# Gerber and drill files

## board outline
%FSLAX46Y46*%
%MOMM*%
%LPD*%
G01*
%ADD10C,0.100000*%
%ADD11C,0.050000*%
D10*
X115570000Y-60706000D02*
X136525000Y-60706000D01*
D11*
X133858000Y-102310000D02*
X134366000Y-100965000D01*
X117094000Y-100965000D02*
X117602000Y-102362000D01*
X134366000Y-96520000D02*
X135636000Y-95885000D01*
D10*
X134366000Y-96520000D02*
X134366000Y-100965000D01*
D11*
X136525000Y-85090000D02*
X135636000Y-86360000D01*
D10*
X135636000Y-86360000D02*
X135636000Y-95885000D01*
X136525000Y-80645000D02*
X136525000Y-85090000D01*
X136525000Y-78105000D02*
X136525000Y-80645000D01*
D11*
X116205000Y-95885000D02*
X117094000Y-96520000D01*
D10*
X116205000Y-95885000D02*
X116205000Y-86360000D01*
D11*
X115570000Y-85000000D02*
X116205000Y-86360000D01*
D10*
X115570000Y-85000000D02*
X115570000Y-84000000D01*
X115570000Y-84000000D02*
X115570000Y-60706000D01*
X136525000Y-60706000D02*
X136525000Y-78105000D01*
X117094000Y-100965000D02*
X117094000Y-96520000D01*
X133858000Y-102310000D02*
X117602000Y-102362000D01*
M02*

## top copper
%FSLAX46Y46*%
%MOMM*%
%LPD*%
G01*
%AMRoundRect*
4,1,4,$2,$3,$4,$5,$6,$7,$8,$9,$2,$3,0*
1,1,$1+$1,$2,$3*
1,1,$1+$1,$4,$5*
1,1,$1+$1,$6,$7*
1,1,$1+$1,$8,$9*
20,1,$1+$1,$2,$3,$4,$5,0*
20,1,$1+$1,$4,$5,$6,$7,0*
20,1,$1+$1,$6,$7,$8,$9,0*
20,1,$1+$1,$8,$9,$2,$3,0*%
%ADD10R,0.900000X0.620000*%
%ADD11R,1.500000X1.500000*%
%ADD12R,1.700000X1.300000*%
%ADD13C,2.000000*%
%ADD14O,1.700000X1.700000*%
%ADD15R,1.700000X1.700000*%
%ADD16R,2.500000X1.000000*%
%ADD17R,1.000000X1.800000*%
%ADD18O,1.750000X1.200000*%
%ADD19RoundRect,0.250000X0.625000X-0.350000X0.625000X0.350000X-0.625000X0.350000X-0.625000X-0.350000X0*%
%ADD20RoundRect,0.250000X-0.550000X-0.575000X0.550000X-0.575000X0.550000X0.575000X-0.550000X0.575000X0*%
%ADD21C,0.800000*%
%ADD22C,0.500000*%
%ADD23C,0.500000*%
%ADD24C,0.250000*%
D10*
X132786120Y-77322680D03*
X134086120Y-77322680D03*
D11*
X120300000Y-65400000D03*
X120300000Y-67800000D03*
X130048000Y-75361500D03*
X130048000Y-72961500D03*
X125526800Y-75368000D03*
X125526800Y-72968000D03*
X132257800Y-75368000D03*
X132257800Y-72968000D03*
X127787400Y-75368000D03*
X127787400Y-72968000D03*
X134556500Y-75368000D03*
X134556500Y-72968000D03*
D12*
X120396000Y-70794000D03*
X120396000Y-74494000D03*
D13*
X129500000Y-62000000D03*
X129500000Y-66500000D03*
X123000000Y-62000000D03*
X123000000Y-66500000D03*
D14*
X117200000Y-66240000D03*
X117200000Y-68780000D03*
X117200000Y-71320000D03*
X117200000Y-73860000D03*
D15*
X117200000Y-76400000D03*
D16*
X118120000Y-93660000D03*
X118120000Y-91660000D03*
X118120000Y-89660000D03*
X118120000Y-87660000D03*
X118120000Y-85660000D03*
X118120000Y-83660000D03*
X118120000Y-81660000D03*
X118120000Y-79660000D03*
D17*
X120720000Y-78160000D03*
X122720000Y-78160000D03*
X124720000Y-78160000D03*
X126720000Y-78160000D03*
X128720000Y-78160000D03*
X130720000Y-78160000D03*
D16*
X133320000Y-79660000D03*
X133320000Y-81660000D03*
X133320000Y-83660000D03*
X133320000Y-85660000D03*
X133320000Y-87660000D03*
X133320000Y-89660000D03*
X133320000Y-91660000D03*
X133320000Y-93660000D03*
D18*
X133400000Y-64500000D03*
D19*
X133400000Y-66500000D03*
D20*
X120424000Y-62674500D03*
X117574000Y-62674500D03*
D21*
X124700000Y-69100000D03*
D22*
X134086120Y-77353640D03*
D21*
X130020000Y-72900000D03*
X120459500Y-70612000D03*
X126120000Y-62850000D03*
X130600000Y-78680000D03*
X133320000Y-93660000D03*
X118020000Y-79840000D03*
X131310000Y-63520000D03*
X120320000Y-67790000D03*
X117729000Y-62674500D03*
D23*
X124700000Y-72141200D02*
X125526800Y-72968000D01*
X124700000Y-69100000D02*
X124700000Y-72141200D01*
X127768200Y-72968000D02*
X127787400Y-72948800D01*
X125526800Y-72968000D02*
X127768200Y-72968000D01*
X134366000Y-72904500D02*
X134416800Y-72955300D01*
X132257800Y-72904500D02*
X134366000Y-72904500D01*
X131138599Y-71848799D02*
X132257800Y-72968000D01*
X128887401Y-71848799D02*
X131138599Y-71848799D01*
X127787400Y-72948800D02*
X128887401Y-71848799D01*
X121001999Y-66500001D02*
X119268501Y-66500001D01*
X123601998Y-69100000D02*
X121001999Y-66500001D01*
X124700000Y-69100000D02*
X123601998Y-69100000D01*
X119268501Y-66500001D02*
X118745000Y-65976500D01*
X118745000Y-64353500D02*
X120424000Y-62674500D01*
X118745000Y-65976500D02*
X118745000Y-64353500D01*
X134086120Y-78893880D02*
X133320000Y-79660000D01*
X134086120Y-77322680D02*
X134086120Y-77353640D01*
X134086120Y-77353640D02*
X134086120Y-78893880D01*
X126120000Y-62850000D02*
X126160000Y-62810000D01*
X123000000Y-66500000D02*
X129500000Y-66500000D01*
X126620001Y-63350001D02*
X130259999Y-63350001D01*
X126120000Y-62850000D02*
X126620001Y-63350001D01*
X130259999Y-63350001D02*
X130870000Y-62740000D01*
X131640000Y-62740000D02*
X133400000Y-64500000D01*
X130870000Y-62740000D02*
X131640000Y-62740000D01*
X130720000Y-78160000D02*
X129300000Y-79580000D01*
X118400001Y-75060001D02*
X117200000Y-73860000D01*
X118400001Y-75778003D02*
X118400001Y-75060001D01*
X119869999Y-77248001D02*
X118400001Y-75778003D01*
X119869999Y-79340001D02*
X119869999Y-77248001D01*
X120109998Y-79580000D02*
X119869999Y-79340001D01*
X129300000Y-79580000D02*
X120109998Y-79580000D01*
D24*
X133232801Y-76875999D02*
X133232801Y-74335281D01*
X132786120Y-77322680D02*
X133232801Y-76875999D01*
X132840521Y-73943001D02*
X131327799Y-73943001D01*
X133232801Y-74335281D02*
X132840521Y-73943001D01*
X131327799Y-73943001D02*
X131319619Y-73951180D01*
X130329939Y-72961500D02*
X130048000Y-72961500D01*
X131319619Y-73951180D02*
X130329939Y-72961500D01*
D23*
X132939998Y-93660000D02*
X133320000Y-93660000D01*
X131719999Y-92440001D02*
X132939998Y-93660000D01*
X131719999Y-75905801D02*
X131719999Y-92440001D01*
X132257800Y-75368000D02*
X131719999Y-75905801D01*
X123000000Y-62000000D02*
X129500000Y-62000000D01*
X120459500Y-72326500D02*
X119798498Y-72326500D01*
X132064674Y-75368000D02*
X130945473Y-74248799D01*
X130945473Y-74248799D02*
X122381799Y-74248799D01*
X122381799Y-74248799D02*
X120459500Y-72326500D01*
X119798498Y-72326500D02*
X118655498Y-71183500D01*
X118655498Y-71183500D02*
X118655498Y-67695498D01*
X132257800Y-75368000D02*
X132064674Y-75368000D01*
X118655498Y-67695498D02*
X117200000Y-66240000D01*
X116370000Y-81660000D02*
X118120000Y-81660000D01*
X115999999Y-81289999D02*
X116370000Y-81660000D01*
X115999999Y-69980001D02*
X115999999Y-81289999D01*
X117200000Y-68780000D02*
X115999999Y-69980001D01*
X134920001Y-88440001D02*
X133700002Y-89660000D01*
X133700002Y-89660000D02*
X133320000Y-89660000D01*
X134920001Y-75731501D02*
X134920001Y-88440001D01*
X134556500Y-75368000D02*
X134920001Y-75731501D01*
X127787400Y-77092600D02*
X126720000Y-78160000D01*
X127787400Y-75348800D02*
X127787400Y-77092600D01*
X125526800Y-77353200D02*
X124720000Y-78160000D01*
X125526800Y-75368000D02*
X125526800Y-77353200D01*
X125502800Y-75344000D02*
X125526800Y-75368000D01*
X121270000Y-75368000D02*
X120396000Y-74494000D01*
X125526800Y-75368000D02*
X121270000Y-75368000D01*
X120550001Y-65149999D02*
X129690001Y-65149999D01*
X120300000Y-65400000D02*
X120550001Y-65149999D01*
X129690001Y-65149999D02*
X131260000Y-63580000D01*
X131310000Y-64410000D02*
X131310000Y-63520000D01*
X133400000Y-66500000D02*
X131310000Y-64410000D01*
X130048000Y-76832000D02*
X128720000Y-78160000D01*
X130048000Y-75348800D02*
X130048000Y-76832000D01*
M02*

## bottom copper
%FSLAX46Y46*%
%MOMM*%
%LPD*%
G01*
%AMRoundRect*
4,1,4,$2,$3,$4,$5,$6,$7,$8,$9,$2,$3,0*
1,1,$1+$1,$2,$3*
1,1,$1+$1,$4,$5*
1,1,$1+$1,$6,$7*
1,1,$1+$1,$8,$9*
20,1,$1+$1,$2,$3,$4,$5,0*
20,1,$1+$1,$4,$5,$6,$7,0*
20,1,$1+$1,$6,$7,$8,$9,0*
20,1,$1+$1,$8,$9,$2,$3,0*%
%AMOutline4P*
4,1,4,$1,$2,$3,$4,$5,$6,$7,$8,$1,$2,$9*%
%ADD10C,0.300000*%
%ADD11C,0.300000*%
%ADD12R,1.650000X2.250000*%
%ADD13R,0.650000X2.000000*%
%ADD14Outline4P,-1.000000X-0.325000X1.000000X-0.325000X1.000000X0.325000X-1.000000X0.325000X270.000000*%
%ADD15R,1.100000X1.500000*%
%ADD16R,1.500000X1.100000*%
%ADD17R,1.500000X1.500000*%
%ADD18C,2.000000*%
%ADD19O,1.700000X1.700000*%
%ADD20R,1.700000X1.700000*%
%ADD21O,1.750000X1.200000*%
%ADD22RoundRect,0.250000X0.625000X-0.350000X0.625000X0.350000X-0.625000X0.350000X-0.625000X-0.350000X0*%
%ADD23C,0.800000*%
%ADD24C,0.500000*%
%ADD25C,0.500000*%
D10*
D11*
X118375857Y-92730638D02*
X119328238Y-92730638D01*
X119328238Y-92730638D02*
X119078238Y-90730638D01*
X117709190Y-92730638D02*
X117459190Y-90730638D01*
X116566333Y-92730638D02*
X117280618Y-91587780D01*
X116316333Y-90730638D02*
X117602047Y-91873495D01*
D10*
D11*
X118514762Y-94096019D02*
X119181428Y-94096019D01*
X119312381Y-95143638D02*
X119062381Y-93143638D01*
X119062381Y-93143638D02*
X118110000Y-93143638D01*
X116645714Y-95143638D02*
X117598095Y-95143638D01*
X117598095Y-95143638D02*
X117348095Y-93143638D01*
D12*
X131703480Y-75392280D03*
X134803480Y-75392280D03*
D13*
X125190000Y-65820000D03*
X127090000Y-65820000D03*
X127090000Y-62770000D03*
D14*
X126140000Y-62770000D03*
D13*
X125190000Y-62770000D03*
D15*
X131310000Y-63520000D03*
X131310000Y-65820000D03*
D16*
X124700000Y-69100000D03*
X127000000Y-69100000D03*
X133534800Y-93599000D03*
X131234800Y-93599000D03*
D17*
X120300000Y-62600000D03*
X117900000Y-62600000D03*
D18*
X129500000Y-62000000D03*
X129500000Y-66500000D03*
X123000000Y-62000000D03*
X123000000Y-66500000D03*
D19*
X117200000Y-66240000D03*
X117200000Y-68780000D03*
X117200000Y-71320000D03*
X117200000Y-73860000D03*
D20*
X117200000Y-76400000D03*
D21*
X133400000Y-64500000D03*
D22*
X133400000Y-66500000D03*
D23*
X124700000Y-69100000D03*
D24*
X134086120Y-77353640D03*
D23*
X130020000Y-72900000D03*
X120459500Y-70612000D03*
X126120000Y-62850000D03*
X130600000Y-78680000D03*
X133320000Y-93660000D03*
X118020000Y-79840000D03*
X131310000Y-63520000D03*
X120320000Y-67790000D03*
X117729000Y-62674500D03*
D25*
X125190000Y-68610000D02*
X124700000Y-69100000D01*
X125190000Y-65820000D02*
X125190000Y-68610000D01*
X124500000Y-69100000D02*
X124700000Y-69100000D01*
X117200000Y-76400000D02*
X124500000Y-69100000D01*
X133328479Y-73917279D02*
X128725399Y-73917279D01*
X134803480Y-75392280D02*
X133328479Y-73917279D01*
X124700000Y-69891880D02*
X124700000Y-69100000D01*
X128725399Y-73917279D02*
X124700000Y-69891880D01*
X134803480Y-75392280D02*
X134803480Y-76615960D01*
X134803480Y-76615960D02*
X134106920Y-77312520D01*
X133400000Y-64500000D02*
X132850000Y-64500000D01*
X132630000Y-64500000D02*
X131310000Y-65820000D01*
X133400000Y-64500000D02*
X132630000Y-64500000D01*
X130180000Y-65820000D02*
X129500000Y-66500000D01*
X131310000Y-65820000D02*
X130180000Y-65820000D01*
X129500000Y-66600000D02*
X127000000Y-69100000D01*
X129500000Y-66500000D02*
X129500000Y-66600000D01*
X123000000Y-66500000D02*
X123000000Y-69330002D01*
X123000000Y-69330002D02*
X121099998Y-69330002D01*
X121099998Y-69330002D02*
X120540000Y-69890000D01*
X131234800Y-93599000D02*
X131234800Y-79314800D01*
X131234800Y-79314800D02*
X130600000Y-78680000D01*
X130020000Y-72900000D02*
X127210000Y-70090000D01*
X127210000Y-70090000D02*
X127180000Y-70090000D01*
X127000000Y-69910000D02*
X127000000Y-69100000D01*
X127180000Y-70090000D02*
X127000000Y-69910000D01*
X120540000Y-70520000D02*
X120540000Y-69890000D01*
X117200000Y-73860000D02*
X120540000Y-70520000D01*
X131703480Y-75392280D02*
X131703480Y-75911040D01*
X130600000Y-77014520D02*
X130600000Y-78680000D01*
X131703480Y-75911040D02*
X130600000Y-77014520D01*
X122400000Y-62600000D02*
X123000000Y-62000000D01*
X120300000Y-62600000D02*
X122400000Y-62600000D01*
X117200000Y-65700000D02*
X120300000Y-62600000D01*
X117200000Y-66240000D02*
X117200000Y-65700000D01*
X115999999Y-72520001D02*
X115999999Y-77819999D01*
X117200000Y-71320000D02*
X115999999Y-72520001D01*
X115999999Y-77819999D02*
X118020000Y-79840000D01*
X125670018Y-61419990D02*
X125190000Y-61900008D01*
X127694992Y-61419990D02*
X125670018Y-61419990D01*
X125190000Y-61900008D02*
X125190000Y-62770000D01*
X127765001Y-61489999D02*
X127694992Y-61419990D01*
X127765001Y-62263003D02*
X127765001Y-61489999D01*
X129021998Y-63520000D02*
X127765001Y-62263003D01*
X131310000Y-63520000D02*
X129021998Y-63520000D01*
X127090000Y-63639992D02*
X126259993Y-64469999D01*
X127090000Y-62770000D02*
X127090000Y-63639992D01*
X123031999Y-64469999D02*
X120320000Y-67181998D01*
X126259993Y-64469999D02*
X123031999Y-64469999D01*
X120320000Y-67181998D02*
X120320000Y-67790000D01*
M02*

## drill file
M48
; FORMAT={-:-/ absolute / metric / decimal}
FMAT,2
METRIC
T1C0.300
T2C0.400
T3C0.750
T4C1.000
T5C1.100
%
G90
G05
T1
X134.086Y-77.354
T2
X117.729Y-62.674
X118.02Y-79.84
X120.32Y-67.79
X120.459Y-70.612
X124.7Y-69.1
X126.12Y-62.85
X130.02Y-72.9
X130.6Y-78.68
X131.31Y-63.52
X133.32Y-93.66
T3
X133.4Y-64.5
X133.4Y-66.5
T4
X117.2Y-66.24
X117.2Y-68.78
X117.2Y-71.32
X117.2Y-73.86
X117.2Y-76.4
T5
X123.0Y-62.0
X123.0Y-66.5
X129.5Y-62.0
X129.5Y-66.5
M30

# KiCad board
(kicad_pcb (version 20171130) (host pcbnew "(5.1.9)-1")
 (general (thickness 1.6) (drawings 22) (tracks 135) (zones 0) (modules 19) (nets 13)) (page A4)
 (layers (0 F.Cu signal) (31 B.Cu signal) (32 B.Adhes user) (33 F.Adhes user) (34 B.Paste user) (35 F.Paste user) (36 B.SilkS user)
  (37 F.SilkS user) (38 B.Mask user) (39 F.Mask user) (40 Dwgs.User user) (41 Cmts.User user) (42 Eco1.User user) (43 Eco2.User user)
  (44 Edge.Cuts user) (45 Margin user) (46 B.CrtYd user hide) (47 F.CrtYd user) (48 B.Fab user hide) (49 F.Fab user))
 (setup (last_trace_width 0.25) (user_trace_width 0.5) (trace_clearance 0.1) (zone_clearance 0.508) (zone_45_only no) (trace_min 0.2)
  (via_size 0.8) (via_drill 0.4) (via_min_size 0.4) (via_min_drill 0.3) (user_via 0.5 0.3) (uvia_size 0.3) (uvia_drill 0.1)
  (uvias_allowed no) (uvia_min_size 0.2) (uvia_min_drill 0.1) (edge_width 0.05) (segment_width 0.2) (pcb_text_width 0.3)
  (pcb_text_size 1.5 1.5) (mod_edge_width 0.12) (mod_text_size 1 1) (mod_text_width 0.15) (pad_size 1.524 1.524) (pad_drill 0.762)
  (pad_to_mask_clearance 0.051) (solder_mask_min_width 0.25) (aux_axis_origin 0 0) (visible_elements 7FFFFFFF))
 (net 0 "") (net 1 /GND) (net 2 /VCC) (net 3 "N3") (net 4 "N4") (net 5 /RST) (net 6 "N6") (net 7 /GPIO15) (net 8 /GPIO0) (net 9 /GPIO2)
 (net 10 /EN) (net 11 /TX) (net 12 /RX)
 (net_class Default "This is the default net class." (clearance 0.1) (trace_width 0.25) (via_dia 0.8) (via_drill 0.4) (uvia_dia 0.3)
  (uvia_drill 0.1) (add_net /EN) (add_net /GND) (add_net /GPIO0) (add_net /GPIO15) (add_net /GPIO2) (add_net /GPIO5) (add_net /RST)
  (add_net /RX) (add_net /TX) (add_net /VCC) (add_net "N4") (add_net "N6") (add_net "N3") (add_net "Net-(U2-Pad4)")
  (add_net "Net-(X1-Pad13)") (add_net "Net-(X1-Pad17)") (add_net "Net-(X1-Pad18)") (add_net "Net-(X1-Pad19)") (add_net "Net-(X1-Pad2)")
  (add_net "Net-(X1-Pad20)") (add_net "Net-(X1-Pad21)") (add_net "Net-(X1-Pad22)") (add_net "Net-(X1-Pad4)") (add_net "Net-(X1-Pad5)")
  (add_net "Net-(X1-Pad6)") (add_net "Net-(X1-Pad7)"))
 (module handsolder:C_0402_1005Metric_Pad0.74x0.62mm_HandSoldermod (layer F.Cu) (at 133.43612 77.32268 180)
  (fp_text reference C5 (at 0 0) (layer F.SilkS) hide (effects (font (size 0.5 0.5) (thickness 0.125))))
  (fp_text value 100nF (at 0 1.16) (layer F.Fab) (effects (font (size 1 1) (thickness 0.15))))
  (pad 2 smd rect (at 0.65 0 180) (size 0.9 0.62) (layers F.Cu F.Paste F.Mask) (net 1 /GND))
  (pad 1 smd rect (at -0.65 0 180) (size 0.9 0.62) (layers F.Cu F.Paste F.Mask) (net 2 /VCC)))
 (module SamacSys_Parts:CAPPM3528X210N (layer B.Cu) (at 133.25348 75.39228 180)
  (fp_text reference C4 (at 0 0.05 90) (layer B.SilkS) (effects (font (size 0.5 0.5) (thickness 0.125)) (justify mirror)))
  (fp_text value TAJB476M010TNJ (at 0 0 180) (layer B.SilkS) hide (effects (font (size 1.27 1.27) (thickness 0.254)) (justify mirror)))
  (pad 2 smd rect (at 1.55 0 180) (size 1.65 2.25) (layers B.Cu B.Paste B.Mask) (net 1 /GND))
  (pad 1 smd rect (at -1.55 0 180) (size 1.65 2.25) (layers B.Cu B.Paste B.Mask) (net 2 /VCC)))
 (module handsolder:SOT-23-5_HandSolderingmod (layer B.Cu) (at 126.14 64.32 270)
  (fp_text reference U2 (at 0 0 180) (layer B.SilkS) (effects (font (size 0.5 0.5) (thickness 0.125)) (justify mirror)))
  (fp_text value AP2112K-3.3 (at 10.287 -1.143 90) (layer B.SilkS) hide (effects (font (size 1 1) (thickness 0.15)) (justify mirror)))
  (pad 5 smd rect (at 1.5 0.95 270) (size 2 0.65) (layers B.Cu B.Paste B.Mask) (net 2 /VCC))
  (pad 4 smd rect (at 1.5 -0.95 270) (size 2 0.65) (layers B.Cu B.Paste B.Mask))
  (pad 3 smd rect (at -1.55 -0.95 270) (size 2 0.65) (layers B.Cu B.Paste B.Mask) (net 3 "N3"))
  (pad 2 smd trapezoid (at -1.55 0 270) (size 2 0.65) (layers B.Cu B.Paste B.Mask) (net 1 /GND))
  (pad 1 smd rect (at -1.55 0.95 270) (size 2 0.65) (layers B.Cu B.Paste B.Mask) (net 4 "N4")))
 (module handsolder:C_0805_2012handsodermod (layer B.Cu) (at 131.31 64.67 90)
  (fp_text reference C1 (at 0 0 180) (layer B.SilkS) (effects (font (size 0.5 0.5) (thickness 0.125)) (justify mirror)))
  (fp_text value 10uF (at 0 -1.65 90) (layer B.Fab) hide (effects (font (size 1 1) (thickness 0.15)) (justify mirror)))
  (pad 2 smd rect (at 1.15 0 90) (size 1.5 1.1) (layers B.Cu B.Paste B.Mask) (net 4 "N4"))
  (pad 1 smd rect (at -1.15 0 90) (size 1.5 1.1) (layers B.Cu B.Paste B.Mask) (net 1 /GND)))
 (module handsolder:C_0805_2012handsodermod (layer B.Cu) (at 125.85 69.1 180)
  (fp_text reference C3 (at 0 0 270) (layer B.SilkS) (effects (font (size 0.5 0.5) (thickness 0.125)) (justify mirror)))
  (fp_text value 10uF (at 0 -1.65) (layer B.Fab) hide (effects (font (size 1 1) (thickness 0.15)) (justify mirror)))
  (pad 2 smd rect (at 1.15 0 180) (size 1.5 1.1) (layers B.Cu B.Paste B.Mask) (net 2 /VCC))
  (pad 1 smd rect (at -1.15 0 180) (size 1.5 1.1) (layers B.Cu B.Paste B.Mask) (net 1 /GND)))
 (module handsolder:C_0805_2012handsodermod (layer B.Cu) (at 132.3848 93.599)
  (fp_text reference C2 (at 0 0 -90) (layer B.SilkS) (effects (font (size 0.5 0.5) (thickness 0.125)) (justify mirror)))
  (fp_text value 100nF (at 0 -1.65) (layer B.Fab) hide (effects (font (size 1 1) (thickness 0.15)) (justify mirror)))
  (pad 2 smd rect (at 1.15 0) (size 1.5 1.1) (layers B.Cu B.Paste B.Mask) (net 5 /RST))
  (pad 1 smd rect (at -1.15 0) (size 1.5 1.1) (layers B.Cu B.Paste B.Mask) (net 1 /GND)))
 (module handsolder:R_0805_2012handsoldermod (layer F.Cu) (at 120.3 66.6 90)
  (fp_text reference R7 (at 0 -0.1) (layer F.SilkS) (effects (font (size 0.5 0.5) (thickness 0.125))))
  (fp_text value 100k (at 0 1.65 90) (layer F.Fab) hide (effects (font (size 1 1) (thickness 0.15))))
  (pad 2 smd rect (at 1.2 0 90) (size 1.5 1.5) (layers F.Cu F.Paste F.Mask) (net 4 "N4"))
  (pad 1 smd rect (at -1.2 0 90) (size 1.5 1.5) (layers F.Cu F.Paste F.Mask) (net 3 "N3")))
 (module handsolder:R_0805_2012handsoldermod (layer B.Cu) (at 119.1 62.6)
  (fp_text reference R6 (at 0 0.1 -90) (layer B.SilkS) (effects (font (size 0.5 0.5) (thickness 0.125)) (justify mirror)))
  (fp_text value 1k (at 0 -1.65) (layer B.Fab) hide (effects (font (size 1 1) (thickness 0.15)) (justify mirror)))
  (pad 2 smd rect (at 1.2 0) (size 1.5 1.5) (layers B.Cu B.Paste B.Mask) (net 5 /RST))
  (pad 1 smd rect (at -1.2 0) (size 1.5 1.5) (layers B.Cu B.Paste B.Mask) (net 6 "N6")))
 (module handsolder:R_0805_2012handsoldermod (layer F.Cu) (at 130.048 74.1615 270)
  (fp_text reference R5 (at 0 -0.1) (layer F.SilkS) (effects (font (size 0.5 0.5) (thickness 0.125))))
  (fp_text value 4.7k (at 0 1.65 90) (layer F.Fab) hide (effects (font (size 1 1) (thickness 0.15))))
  (pad 2 smd rect (at 1.2 0 270) (size 1.5 1.5) (layers F.Cu F.Paste F.Mask) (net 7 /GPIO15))
  (pad 1 smd rect (at -1.2 0 270) (size 1.5 1.5) (layers F.Cu F.Paste F.Mask) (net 1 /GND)))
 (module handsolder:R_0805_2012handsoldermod (layer F.Cu) (at 125.5268 74.168 270)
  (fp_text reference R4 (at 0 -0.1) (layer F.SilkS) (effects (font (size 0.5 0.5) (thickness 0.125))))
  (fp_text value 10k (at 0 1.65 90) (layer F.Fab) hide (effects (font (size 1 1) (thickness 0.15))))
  (pad 2 smd rect (at 1.2 0 270) (size 1.5 1.5) (layers F.Cu F.Paste F.Mask) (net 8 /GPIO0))
  (pad 1 smd rect (at -1.2 0 270) (size 1.5 1.5) (layers F.Cu F.Paste F.Mask) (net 2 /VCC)))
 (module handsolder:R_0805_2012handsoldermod (layer F.Cu) (at 132.2578 74.168 270)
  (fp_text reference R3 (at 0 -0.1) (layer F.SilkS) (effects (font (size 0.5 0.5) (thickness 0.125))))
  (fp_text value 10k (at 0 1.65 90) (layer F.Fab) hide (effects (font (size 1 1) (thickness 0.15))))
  (pad 2 smd rect (at 1.2 0 270) (size 1.5 1.5) (layers F.Cu F.Paste F.Mask) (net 5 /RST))
  (pad 1 smd rect (at -1.2 0 270) (size 1.5 1.5) (layers F.Cu F.Paste F.Mask) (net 2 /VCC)))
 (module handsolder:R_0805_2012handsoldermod (layer F.Cu) (at 127.7874 74.168 270)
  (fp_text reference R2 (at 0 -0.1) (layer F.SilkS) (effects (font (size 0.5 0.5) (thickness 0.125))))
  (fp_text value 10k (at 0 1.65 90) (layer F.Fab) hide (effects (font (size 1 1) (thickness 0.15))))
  (pad 2 smd rect (at 1.2 0 270) (size 1.5 1.5) (layers F.Cu F.Paste F.Mask) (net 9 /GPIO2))
  (pad 1 smd rect (at -1.2 0 270) (size 1.5 1.5) (layers F.Cu F.Paste F.Mask) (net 2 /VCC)))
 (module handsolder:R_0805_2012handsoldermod (layer F.Cu) (at 134.5565 74.168 270)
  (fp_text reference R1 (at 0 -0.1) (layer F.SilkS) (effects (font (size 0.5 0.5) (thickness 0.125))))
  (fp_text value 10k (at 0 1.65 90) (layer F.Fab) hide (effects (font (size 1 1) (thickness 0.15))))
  (pad 2 smd rect (at 1.2 0 270) (size 1.5 1.5) (layers F.Cu F.Paste F.Mask) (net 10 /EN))
  (pad 1 smd rect (at -1.2 0 270) (size 1.5 1.5) (layers F.Cu F.Paste F.Mask) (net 2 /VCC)))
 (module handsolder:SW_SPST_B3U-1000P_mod (layer F.Cu) (at 120.396 72.644 90)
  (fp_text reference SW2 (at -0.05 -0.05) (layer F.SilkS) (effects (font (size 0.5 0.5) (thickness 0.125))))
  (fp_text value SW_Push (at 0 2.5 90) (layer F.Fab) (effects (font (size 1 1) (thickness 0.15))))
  (pad 2 smd rect (at 1.85 0 90) (size 1.3 1.7) (layers F.Cu F.Paste F.Mask) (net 1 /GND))
  (pad 1 smd rect (at -1.85 0 90) (size 1.3 1.7) (layers F.Cu F.Paste F.Mask) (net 8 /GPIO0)))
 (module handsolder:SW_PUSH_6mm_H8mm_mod (layer F.Cu) (at 123 62)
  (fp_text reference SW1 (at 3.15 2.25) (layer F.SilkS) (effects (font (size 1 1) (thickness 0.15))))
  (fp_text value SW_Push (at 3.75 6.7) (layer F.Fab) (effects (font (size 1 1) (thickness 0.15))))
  (pad 1 thru_hole circle (at 6.5 0 90) (size 2 2) (drill 1.1) (layers *.Cu *.Mask) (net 5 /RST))
  (pad 2 thru_hole circle (at 6.5 4.5 90) (size 2 2) (drill 1.1) (layers *.Cu *.Mask) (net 1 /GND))
  (pad 1 thru_hole circle (at 0 0 90) (size 2 2) (drill 1.1) (layers *.Cu *.Mask) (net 5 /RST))
  (pad 2 thru_hole circle (at 0 4.5 90) (size 2 2) (drill 1.1) (layers *.Cu *.Mask) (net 1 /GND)))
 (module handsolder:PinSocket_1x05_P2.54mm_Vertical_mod (layer F.Cu) (at 117.2 76.4 180)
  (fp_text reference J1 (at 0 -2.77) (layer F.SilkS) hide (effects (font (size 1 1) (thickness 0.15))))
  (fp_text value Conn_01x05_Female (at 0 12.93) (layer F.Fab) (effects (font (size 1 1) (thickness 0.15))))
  (pad 5 thru_hole oval (at 0 10.16 180) (size 1.7 1.7) (drill 1) (layers *.Cu *.Mask) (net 5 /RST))
  (pad 4 thru_hole oval (at 0 7.62 180) (size 1.7 1.7) (drill 1) (layers *.Cu *.Mask) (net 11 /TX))
  (pad 3 thru_hole oval (at 0 5.08 180) (size 1.7 1.7) (drill 1) (layers *.Cu *.Mask) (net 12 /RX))
  (pad 2 thru_hole oval (at 0 2.54 180) (size 1.7 1.7) (drill 1) (layers *.Cu *.Mask) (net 1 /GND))
  (pad 1 thru_hole rect (at 0 0 180) (size 1.7 1.7) (drill 1) (layers *.Cu *.Mask) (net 2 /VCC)))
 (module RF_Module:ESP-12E (layer F.Cu) (at 125.72 90.16 180)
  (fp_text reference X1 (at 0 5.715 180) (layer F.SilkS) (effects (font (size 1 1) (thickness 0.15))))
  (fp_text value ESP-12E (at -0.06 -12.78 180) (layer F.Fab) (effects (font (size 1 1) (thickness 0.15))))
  (pad 22 smd rect (at 7.6 -3.5 180) (size 2.5 1) (layers F.Cu F.Paste F.Mask))
  (pad 21 smd rect (at 7.6 -1.5 180) (size 2.5 1) (layers F.Cu F.Paste F.Mask))
  (pad 20 smd rect (at 7.6 0.5 180) (size 2.5 1) (layers F.Cu F.Paste F.Mask))
  (pad 19 smd rect (at 7.6 2.5 180) (size 2.5 1) (layers F.Cu F.Paste F.Mask))
  (pad 18 smd rect (at 7.6 4.5 180) (size 2.5 1) (layers F.Cu F.Paste F.Mask))
  (pad 17 smd rect (at 7.6 6.5 180) (size 2.5 1) (layers F.Cu F.Paste F.Mask))
  (pad 16 smd rect (at 7.6 8.5 180) (size 2.5 1) (layers F.Cu F.Paste F.Mask) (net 11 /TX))
  (pad 15 smd rect (at 7.6 10.5 180) (size 2.5 1) (layers F.Cu F.Paste F.Mask) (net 12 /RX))
  (pad 14 smd rect (at 5 12 180) (size 1 1.8) (layers F.Cu F.Paste F.Mask))
  (pad 13 smd rect (at 3 12 180) (size 1 1.8) (layers F.Cu F.Paste F.Mask))
  (pad 12 smd rect (at 1 12 180) (size 1 1.8) (layers F.Cu F.Paste F.Mask) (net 8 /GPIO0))
  (pad 11 smd rect (at -1 12 180) (size 1 1.8) (layers F.Cu F.Paste F.Mask) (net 9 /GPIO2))
  (pad 10 smd rect (at -3 12 180) (size 1 1.8) (layers F.Cu F.Paste F.Mask) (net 7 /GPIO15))
  (pad 9 smd rect (at -5 12 180) (size 1 1.8) (layers F.Cu F.Paste F.Mask) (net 1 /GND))
  (pad 8 smd rect (at -7.6 10.5 180) (size 2.5 1) (layers F.Cu F.Paste F.Mask) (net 2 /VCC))
  (pad 7 smd rect (at -7.6 8.5 180) (size 2.5 1) (layers F.Cu F.Paste F.Mask))
  (pad 6 smd rect (at -7.6 6.5 180) (size 2.5 1) (layers F.Cu F.Paste F.Mask))
  (pad 5 smd rect (at -7.6 4.5 180) (size 2.5 1) (layers F.Cu F.Paste F.Mask))
  (pad 4 smd rect (at -7.6 2.5 180) (size 2.5 1) (layers F.Cu F.Paste F.Mask))
  (pad 3 smd rect (at -7.6 0.5 180) (size 2.5 1) (layers F.Cu F.Paste F.Mask) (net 10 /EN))
  (pad 2 smd rect (at -7.6 -1.5 180) (size 2.5 1) (layers F.Cu F.Paste F.Mask))
  (pad 1 smd rect (at -7.6 -3.5 180) (size 2.5 1) (layers F.Cu F.Paste F.Mask) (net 5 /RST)))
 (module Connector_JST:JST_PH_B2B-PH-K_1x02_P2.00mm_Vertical (layer F.Cu) (at 133.4 66.5 90)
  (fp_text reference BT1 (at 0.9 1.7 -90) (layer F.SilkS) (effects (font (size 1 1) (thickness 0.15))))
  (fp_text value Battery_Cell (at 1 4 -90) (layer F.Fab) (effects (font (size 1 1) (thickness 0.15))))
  (pad 2 thru_hole oval (at 2 0 90) (size 1.2 1.75) (drill 0.75) (layers *.Cu *.Mask) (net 1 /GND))
  (pad 1 thru_hole roundrect (at 0 0 90) (size 1.2 1.75) (drill 0.75) (layers *.Cu *.Mask) (roundrect_rratio 0.208333) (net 4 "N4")))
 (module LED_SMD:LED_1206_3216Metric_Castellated (layer F.Cu) (at 118.999 62.6745)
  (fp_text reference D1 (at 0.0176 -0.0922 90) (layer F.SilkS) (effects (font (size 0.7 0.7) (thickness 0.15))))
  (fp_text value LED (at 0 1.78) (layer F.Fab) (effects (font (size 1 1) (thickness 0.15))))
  (pad 2 smd roundrect (at 1.425 0) (size 1.6 1.65) (layers F.Cu F.Paste F.Mask) (roundrect_rratio 0.15625) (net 2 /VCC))
  (pad 1 smd roundrect (at -1.425 0) (size 1.6 1.65) (layers F.Cu F.Paste F.Mask) (roundrect_rratio 0.15625) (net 6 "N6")))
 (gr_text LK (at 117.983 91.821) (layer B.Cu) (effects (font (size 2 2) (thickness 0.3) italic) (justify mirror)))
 (gr_line (start 115.57 60.706) (end 136.525 60.706) (layer Edge.Cuts) (width 0.1))
 (gr_line (start 133.858 102.31) (end 134.366 100.965) (layer Edge.Cuts) (width 0.05))
 (gr_line (start 117.094 100.965) (end 117.602 102.362) (layer Edge.Cuts) (width 0.05))
 (gr_line (start 134.366 96.52) (end 135.636 95.885) (layer Edge.Cuts) (width 0.05))
 (gr_line (start 134.366 96.52) (end 134.366 100.965) (layer Edge.Cuts) (width 0.1))
 (gr_line (start 136.525 85.09) (end 135.636 86.36) (layer Edge.Cuts) (width 0.05))
 (gr_line (start 135.636 86.36) (end 135.636 95.885) (layer Edge.Cuts) (width 0.1))
 (gr_line (start 136.525 80.645) (end 136.525 85.09) (layer Edge.Cuts) (width 0.1))
 (gr_line (start 136.525 78.105) (end 136.525 80.645) (layer Edge.Cuts) (width 0.1))
 (gr_line (start 116.205 95.885) (end 117.094 96.52) (layer Edge.Cuts) (width 0.05))
 (gr_line (start 116.205 95.885) (end 116.205 86.36) (layer Edge.Cuts) (width 0.1))
 (gr_line (start 115.57 85) (end 116.205 86.36) (layer Edge.Cuts) (width 0.05))
 (gr_line (start 115.57 85) (end 115.57 84) (layer Edge.Cuts) (width 0.1))
 (gr_line (start 115.57 84) (end 115.57 60.706) (layer Edge.Cuts) (width 0.1))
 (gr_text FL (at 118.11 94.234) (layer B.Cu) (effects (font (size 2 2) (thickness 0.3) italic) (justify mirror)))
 (gr_line (start 136.525 60.706) (end 136.525 78.105) (layer Edge.Cuts) (width 0.1))
 (gr_line (start 117.094 100.965) (end 117.094 96.52) (layer Edge.Cuts) (width 0.1))
 (gr_line (start 133.858 102.31) (end 117.602 102.362) (layer Edge.Cuts) (width 0.1))
 (segment (start 125.19 68.61) (end 124.7 69.1) (width 0.5) (layer B.Cu) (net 2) (status 30))
 (segment (start 125.19 65.82) (end 125.19 68.61) (width 0.5) (layer B.Cu) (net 2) (status 30))
 (via (at 124.7 69.1) (size 0.8) (drill 0.4) (layers F.Cu B.Cu) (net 2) (status 30))
 (segment (start 124.7 72.1412) (end 125.5268 72.968) (width 0.5) (layer F.Cu) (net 2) (status 20))
 (segment (start 124.7 69.1) (end 124.7 72.1412) (width 0.5) (layer F.Cu) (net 2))
 (segment (start 127.7682 72.968) (end 127.7874 72.9488) (width 0.5) (layer F.Cu) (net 2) (status 30))
 (segment (start 125.5268 72.968) (end 127.7682 72.968) (width 0.5) (layer F.Cu) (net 2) (status 30))
 (segment (start 134.366 72.9045) (end 134.4168 72.9553) (width 0.5) (layer F.Cu) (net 2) (status 30))
 (segment (start 132.2578 72.9045) (end 134.366 72.9045) (width 0.5) (layer F.Cu) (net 2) (status 30))
 (segment (start 131.138599 71.848799) (end 132.2578 72.968) (width 0.5) (layer F.Cu) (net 2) (status 20))
 (segment (start 128.887401 71.848799) (end 131.138599 71.848799) (width 0.5) (layer F.Cu) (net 2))
 (segment (start 127.7874 72.9488) (end 128.887401 71.848799) (width 0.5) (layer F.Cu) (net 2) (status 10))
 (segment (start 124.5 69.1) (end 124.7 69.1) (width 0.5) (layer B.Cu) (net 2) (status 30))
 (segment (start 117.2 76.4) (end 124.5 69.1) (width 0.5) (layer B.Cu) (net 2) (status 30))
 (segment (start 121.001999 66.500001) (end 119.268501 66.500001) (width 0.5) (layer F.Cu) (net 2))
 (segment (start 123.601998 69.1) (end 121.001999 66.500001) (width 0.5) (layer F.Cu) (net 2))
 (segment (start 124.7 69.1) (end 123.601998 69.1) (width 0.5) (layer F.Cu) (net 2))
 (segment (start 119.268501 66.500001) (end 118.745 65.9765) (width 0.5) (layer F.Cu) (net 2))
 (segment (start 118.745 64.3535) (end 120.424 62.6745) (width 0.5) (layer F.Cu) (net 2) (status 20))
 (segment (start 118.745 65.9765) (end 118.745 64.3535) (width 0.5) (layer F.Cu) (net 2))
 (segment (start 133.328479 73.917279) (end 128.725399 73.917279) (width 0.5) (layer B.Cu) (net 2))
 (segment (start 134.80348 75.39228) (end 133.328479 73.917279) (width 0.5) (layer B.Cu) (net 2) (status 10))
 (segment (start 124.7 69.89188) (end 124.7 69.1) (width 0.5) (layer B.Cu) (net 2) (status 20))
 (segment (start 128.725399 73.917279) (end 124.7 69.89188) (width 0.5) (layer B.Cu) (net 2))
 (segment (start 134.08612 78.89388) (end 133.32 79.66) (width 0.5) (layer F.Cu) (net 2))
 (segment (start 134.08612 77.32268) (end 134.08612 77.35364) (width 0.5) (layer F.Cu) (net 2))
 (segment (start 134.80348 75.39228) (end 134.80348 76.61596) (width 0.5) (layer B.Cu) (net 2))
 (segment (start 134.80348 76.61596) (end 134.10692 77.31252) (width 0.5) (layer B.Cu) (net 2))
 (segment (start 134.08612 77.35364) (end 134.08612 78.89388) (width 0.5) (layer F.Cu) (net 2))
 (via (at 134.08612 77.35364) (size 0.5) (drill 0.3) (layers F.Cu B.Cu) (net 2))
 (via (at 130.02 72.9) (size 0.8) (drill 0.4) (layers F.Cu B.Cu) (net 1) (status 30))
 (segment (start 133.4 64.5) (end 132.85 64.5) (width 0.5) (layer B.Cu) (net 1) (status 30))
 (segment (start 132.63 64.5) (end 131.31 65.82) (width 0.5) (layer B.Cu) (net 1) (status 30))
 (segment (start 133.4 64.5) (end 132.63 64.5) (width 0.5) (layer B.Cu) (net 1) (status 30))
 (segment (start 130.18 65.82) (end 129.5 66.5) (width 0.5) (layer B.Cu) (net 1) (status 30))
 (segment (start 131.31 65.82) (end 130.18 65.82) (width 0.5) (layer B.Cu) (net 1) (status 30))
 (segment (start 129.5 66.6) (end 127 69.1) (width 0.5) (layer B.Cu) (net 1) (status 30))
 (segment (start 129.5 66.5) (end 129.5 66.6) (width 0.5) (layer B.Cu) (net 1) (status 30))
 (segment (start 123 66.5) (end 123 69.330002) (width 0.5) (layer B.Cu) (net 1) (status 10))
 (segment (start 123 69.330002) (end 121.099998 69.330002) (width 0.5) (layer B.Cu) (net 1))
 (segment (start 121.099998 69.330002) (end 120.54 69.89) (width 0.5) (layer B.Cu) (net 1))
 (via (at 120.4595 70.612) (size 0.8) (drill 0.4) (layers F.Cu B.Cu) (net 1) (status 30))
 (segment (start 126.12 62.85) (end 126.16 62.81) (width 0.5) (layer F.Cu) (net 1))
 (via (at 126.12 62.85) (size 0.8) (drill 0.4) (layers F.Cu B.Cu) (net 1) (status 30))
 (segment (start 123 66.5) (end 129.5 66.5) (width 0.5) (layer F.Cu) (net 1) (status 30))
 (segment (start 126.620001 63.350001) (end 130.259999 63.350001) (width 0.5) (layer F.Cu) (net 1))
 (segment (start 126.12 62.85) (end 126.620001 63.350001) (width 0.5) (layer F.Cu) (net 1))
 (segment (start 130.259999 63.350001) (end 130.87 62.74) (width 0.5) (layer F.Cu) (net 1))
 (segment (start 131.64 62.74) (end 133.4 64.5) (width 0.5) (layer F.Cu) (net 1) (status 20))
 (segment (start 130.87 62.74) (end 131.64 62.74) (width 0.5) (layer F.Cu) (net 1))
 (segment (start 131.2348 93.599) (end 131.2348 79.3148) (width 0.5) (layer B.Cu) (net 1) (status 10))
 (segment (start 131.2348 79.3148) (end 130.6 78.68) (width 0.5) (layer B.Cu) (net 1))
 (via (at 130.6 78.68) (size 0.8) (drill 0.4) (layers F.Cu B.Cu) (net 1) (status 30))
 (segment (start 130.72 78.16) (end 129.3 79.58) (width 0.5) (layer F.Cu) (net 1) (status 10))
 (segment (start 118.400001 75.060001) (end 117.2 73.86) (width 0.5) (layer F.Cu) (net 1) (status 20))
 (segment (start 118.400001 75.778003) (end 118.400001 75.060001) (width 0.5) (layer F.Cu) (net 1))
 (segment (start 119.869999 77.248001) (end 118.400001 75.778003) (width 0.5) (layer F.Cu) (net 1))
 (segment (start 119.869999 79.340001) (end 119.869999 77.248001) (width 0.5) (layer F.Cu) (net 1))
 (segment (start 120.109998 79.58) (end 119.869999 79.340001) (width 0.5) (layer F.Cu) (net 1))
 (segment (start 129.3 79.58) (end 120.109998 79.58) (width 0.5) (layer F.Cu) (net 1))
 (segment (start 130.02 72.9) (end 127.21 70.09) (width 0.5) (layer B.Cu) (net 1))
 (segment (start 127.21 70.09) (end 127.18 70.09) (width 0.5) (layer B.Cu) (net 1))
 (segment (start 127 69.91) (end 127 69.1) (width 0.5) (layer B.Cu) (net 1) (status 20))
 (segment (start 127.18 70.09) (end 127 69.91) (width 0.5) (layer B.Cu) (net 1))
 (segment (start 120.54 70.52) (end 120.54 69.89) (width 0.5) (layer B.Cu) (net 1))
 (segment (start 117.2 73.86) (end 120.54 70.52) (width 0.5) (layer B.Cu) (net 1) (status 10))
 (segment (start 131.70348 75.39228) (end 131.70348 75.91104) (width 0.5) (layer B.Cu) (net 1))
 (segment (start 130.6 77.01452) (end 130.6 78.68) (width 0.5) (layer B.Cu) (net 1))
 (segment (start 131.70348 75.91104) (end 130.6 77.01452) (width 0.5) (layer B.Cu) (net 1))
 (segment (start 133.232801 76.875999) (end 133.232801 74.335281) (width 0.25) (layer F.Cu) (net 1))
 (segment (start 132.78612 77.32268) (end 133.232801 76.875999) (width 0.25) (layer F.Cu) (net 1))
 (segment (start 132.840521 73.943001) (end 131.327799 73.943001) (width 0.25) (layer F.Cu) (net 1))
 (segment (start 133.232801 74.335281) (end 132.840521 73.943001) (width 0.25) (layer F.Cu) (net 1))
 (segment (start 131.327799 73.943001) (end 131.319619 73.95118) (width 0.25) (layer F.Cu) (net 1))
 (segment (start 130.329939 72.9615) (end 130.048 72.9615) (width 0.25) (layer F.Cu) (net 1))
 (segment (start 131.319619 73.95118) (end 130.329939 72.9615) (width 0.25) (layer F.Cu) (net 1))
 (segment (start 132.939998 93.66) (end 133.32 93.66) (width 0.5) (layer F.Cu) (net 5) (status 30))
 (segment (start 131.719999 92.440001) (end 132.939998 93.66) (width 0.5) (layer F.Cu) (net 5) (status 20))
 (segment (start 131.719999 75.905801) (end 131.719999 92.440001) (width 0.5) (layer F.Cu) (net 5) (status 10))
 (segment (start 132.2578 75.368) (end 131.719999 75.905801) (width 0.5) (layer F.Cu) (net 5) (status 30))
 (via (at 133.32 93.66) (size 0.8) (drill 0.4) (layers F.Cu B.Cu) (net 5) (status 30))
 (segment (start 122.4 62.6) (end 123 62) (width 0.5) (layer B.Cu) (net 5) (status 30))
 (segment (start 120.3 62.6) (end 122.4 62.6) (width 0.5) (layer B.Cu) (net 5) (status 30))
 (segment (start 123 62) (end 129.5 62) (width 0.5) (layer F.Cu) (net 5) (status 30))
 (segment (start 117.2 65.7) (end 120.3 62.6) (width 0.5) (layer B.Cu) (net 5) (status 30))
 (segment (start 117.2 66.24) (end 117.2 65.7) (width 0.5) (layer B.Cu) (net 5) (status 30))
 (segment (start 120.4595 72.3265) (end 119.798498 72.3265) (width 0.5) (layer F.Cu) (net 5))
 (segment (start 132.064674 75.368) (end 130.945473 74.248799) (width 0.5) (layer F.Cu) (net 5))
 (segment (start 130.945473 74.248799) (end 122.381799 74.248799) (width 0.5) (layer F.Cu) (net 5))
 (segment (start 122.381799 74.248799) (end 120.4595 72.3265) (width 0.5) (layer F.Cu) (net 5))
 (segment (start 119.798498 72.3265) (end 118.655498 71.1835) (width 0.5) (layer F.Cu) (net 5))
 (segment (start 118.655498 71.1835) (end 118.655498 67.695498) (width 0.5) (layer F.Cu) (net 5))
 (segment (start 132.2578 75.368) (end 132.064674 75.368) (width 0.5) (layer F.Cu) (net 5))
 (segment (start 118.655498 67.695498) (end 117.2 66.24) (width 0.5) (layer F.Cu) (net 5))
 (segment (start 115.999999 72.520001) (end 115.999999 77.819999) (width 0.5) (layer B.Cu) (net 12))
 (segment (start 117.2 71.32) (end 115.999999 72.520001) (width 0.5) (layer B.Cu) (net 12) (status 10))
 (segment (start 115.999999 77.819999) (end 118.02 79.84) (width 0.5) (layer B.Cu) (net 12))
 (via (at 118.02 79.84) (size 0.8) (drill 0.4) (layers F.Cu B.Cu) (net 12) (status 30))
 (segment (start 116.37 81.66) (end 118.12 81.66) (width 0.5) (layer F.Cu) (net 11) (status 20))
 (segment (start 115.999999 81.289999) (end 116.37 81.66) (width 0.5) (layer F.Cu) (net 11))
 (segment (start 115.999999 69.980001) (end 115.999999 81.289999) (width 0.5) (layer F.Cu) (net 11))
 (segment (start 117.2 68.78) (end 115.999999 69.980001) (width 0.5) (layer F.Cu) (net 11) (status 10))
 (segment (start 134.920001 88.440001) (end 133.700002 89.66) (width 0.5) (layer F.Cu) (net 10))
 (segment (start 133.700002 89.66) (end 133.32 89.66) (width 0.5) (layer F.Cu) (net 10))
 (segment (start 134.920001 75.731501) (end 134.920001 88.440001) (width 0.5) (layer F.Cu) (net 10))
 (segment (start 134.5565 75.368) (end 134.920001 75.731501) (width 0.5) (layer F.Cu) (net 10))
 (segment (start 127.7874 77.0926) (end 126.72 78.16) (width 0.5) (layer F.Cu) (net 9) (status 20))
 (segment (start 127.7874 75.3488) (end 127.7874 77.0926) (width 0.5) (layer F.Cu) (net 9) (status 10))
 (segment (start 125.5268 77.3532) (end 124.72 78.16) (width 0.5) (layer F.Cu) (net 8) (status 20))
 (segment (start 125.5268 75.368) (end 125.5268 77.3532) (width 0.5) (layer F.Cu) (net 8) (status 10))
 (segment (start 125.5028 75.344) (end 125.5268 75.368) (width 0.5) (layer F.Cu) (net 8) (status 30))
 (segment (start 121.27 75.368) (end 120.396 74.494) (width 0.5) (layer F.Cu) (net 8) (status 20))
 (segment (start 125.5268 75.368) (end 121.27 75.368) (width 0.5) (layer F.Cu) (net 8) (status 10))
 (segment (start 125.670018 61.41999) (end 125.19 61.900008) (width 0.5) (layer B.Cu) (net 4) (status 20))
 (segment (start 127.694992 61.41999) (end 125.670018 61.41999) (width 0.5) (layer B.Cu) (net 4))
 (segment (start 125.19 61.900008) (end 125.19 62.77) (width 0.5) (layer B.Cu) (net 4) (status 30))
 (segment (start 127.765001 61.489999) (end 127.694992 61.41999) (width 0.5) (layer B.Cu) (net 4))
 (segment (start 127.765001 62.263003) (end 127.765001 61.489999) (width 0.5) (layer B.Cu) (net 4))
 (segment (start 129.021998 63.52) (end 127.765001 62.263003) (width 0.5) (layer B.Cu) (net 4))
 (segment (start 120.550001 65.149999) (end 129.690001 65.149999) (width 0.5) (layer F.Cu) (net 4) (status 10))
 (segment (start 120.3 65.4) (end 120.550001 65.149999) (width 0.5) (layer F.Cu) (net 4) (status 30))
 (segment (start 129.690001 65.149999) (end 131.26 63.58) (width 0.5) (layer F.Cu) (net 4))
 (segment (start 131.31 63.52) (end 129.021998 63.52) (width 0.5) (layer B.Cu) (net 4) (status 10))
 (via (at 131.31 63.52) (size 0.8) (drill 0.4) (layers F.Cu B.Cu) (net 4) (status 30))
 (segment (start 131.31 64.41) (end 131.31 63.52) (width 0.5) (layer F.Cu) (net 4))
 (segment (start 133.4 66.5) (end 131.31 64.41) (width 0.5) (layer F.Cu) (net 4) (status 10))
 (segment (start 130.048 76.832) (end 128.72 78.16) (width 0.5) (layer F.Cu) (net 7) (status 20))
 (segment (start 130.048 75.3488) (end 130.048 76.832) (width 0.5) (layer F.Cu) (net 7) (status 10))
 (segment (start 127.09 63.639992) (end 126.259993 64.469999) (width 0.5) (layer B.Cu) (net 3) (status 10))
 (segment (start 127.09 62.77) (end 127.09 63.639992) (width 0.5) (layer B.Cu) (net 3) (status 30))
 (segment (start 123.031999 64.469999) (end 120.32 67.181998) (width 0.5) (layer B.Cu) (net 3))
 (segment (start 126.259993 64.469999) (end 123.031999 64.469999) (width 0.5) (layer B.Cu) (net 3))
 (segment (start 120.32 67.181998) (end 120.32 67.79) (width 0.5) (layer B.Cu) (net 3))
 (via (at 120.32 67.79) (size 0.8) (drill 0.4) (layers F.Cu B.Cu) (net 3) (status 30))
 (via (at 117.729 62.6745) (size 0.8) (drill 0.4) (layers F.Cu B.Cu) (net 6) (status 30)))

